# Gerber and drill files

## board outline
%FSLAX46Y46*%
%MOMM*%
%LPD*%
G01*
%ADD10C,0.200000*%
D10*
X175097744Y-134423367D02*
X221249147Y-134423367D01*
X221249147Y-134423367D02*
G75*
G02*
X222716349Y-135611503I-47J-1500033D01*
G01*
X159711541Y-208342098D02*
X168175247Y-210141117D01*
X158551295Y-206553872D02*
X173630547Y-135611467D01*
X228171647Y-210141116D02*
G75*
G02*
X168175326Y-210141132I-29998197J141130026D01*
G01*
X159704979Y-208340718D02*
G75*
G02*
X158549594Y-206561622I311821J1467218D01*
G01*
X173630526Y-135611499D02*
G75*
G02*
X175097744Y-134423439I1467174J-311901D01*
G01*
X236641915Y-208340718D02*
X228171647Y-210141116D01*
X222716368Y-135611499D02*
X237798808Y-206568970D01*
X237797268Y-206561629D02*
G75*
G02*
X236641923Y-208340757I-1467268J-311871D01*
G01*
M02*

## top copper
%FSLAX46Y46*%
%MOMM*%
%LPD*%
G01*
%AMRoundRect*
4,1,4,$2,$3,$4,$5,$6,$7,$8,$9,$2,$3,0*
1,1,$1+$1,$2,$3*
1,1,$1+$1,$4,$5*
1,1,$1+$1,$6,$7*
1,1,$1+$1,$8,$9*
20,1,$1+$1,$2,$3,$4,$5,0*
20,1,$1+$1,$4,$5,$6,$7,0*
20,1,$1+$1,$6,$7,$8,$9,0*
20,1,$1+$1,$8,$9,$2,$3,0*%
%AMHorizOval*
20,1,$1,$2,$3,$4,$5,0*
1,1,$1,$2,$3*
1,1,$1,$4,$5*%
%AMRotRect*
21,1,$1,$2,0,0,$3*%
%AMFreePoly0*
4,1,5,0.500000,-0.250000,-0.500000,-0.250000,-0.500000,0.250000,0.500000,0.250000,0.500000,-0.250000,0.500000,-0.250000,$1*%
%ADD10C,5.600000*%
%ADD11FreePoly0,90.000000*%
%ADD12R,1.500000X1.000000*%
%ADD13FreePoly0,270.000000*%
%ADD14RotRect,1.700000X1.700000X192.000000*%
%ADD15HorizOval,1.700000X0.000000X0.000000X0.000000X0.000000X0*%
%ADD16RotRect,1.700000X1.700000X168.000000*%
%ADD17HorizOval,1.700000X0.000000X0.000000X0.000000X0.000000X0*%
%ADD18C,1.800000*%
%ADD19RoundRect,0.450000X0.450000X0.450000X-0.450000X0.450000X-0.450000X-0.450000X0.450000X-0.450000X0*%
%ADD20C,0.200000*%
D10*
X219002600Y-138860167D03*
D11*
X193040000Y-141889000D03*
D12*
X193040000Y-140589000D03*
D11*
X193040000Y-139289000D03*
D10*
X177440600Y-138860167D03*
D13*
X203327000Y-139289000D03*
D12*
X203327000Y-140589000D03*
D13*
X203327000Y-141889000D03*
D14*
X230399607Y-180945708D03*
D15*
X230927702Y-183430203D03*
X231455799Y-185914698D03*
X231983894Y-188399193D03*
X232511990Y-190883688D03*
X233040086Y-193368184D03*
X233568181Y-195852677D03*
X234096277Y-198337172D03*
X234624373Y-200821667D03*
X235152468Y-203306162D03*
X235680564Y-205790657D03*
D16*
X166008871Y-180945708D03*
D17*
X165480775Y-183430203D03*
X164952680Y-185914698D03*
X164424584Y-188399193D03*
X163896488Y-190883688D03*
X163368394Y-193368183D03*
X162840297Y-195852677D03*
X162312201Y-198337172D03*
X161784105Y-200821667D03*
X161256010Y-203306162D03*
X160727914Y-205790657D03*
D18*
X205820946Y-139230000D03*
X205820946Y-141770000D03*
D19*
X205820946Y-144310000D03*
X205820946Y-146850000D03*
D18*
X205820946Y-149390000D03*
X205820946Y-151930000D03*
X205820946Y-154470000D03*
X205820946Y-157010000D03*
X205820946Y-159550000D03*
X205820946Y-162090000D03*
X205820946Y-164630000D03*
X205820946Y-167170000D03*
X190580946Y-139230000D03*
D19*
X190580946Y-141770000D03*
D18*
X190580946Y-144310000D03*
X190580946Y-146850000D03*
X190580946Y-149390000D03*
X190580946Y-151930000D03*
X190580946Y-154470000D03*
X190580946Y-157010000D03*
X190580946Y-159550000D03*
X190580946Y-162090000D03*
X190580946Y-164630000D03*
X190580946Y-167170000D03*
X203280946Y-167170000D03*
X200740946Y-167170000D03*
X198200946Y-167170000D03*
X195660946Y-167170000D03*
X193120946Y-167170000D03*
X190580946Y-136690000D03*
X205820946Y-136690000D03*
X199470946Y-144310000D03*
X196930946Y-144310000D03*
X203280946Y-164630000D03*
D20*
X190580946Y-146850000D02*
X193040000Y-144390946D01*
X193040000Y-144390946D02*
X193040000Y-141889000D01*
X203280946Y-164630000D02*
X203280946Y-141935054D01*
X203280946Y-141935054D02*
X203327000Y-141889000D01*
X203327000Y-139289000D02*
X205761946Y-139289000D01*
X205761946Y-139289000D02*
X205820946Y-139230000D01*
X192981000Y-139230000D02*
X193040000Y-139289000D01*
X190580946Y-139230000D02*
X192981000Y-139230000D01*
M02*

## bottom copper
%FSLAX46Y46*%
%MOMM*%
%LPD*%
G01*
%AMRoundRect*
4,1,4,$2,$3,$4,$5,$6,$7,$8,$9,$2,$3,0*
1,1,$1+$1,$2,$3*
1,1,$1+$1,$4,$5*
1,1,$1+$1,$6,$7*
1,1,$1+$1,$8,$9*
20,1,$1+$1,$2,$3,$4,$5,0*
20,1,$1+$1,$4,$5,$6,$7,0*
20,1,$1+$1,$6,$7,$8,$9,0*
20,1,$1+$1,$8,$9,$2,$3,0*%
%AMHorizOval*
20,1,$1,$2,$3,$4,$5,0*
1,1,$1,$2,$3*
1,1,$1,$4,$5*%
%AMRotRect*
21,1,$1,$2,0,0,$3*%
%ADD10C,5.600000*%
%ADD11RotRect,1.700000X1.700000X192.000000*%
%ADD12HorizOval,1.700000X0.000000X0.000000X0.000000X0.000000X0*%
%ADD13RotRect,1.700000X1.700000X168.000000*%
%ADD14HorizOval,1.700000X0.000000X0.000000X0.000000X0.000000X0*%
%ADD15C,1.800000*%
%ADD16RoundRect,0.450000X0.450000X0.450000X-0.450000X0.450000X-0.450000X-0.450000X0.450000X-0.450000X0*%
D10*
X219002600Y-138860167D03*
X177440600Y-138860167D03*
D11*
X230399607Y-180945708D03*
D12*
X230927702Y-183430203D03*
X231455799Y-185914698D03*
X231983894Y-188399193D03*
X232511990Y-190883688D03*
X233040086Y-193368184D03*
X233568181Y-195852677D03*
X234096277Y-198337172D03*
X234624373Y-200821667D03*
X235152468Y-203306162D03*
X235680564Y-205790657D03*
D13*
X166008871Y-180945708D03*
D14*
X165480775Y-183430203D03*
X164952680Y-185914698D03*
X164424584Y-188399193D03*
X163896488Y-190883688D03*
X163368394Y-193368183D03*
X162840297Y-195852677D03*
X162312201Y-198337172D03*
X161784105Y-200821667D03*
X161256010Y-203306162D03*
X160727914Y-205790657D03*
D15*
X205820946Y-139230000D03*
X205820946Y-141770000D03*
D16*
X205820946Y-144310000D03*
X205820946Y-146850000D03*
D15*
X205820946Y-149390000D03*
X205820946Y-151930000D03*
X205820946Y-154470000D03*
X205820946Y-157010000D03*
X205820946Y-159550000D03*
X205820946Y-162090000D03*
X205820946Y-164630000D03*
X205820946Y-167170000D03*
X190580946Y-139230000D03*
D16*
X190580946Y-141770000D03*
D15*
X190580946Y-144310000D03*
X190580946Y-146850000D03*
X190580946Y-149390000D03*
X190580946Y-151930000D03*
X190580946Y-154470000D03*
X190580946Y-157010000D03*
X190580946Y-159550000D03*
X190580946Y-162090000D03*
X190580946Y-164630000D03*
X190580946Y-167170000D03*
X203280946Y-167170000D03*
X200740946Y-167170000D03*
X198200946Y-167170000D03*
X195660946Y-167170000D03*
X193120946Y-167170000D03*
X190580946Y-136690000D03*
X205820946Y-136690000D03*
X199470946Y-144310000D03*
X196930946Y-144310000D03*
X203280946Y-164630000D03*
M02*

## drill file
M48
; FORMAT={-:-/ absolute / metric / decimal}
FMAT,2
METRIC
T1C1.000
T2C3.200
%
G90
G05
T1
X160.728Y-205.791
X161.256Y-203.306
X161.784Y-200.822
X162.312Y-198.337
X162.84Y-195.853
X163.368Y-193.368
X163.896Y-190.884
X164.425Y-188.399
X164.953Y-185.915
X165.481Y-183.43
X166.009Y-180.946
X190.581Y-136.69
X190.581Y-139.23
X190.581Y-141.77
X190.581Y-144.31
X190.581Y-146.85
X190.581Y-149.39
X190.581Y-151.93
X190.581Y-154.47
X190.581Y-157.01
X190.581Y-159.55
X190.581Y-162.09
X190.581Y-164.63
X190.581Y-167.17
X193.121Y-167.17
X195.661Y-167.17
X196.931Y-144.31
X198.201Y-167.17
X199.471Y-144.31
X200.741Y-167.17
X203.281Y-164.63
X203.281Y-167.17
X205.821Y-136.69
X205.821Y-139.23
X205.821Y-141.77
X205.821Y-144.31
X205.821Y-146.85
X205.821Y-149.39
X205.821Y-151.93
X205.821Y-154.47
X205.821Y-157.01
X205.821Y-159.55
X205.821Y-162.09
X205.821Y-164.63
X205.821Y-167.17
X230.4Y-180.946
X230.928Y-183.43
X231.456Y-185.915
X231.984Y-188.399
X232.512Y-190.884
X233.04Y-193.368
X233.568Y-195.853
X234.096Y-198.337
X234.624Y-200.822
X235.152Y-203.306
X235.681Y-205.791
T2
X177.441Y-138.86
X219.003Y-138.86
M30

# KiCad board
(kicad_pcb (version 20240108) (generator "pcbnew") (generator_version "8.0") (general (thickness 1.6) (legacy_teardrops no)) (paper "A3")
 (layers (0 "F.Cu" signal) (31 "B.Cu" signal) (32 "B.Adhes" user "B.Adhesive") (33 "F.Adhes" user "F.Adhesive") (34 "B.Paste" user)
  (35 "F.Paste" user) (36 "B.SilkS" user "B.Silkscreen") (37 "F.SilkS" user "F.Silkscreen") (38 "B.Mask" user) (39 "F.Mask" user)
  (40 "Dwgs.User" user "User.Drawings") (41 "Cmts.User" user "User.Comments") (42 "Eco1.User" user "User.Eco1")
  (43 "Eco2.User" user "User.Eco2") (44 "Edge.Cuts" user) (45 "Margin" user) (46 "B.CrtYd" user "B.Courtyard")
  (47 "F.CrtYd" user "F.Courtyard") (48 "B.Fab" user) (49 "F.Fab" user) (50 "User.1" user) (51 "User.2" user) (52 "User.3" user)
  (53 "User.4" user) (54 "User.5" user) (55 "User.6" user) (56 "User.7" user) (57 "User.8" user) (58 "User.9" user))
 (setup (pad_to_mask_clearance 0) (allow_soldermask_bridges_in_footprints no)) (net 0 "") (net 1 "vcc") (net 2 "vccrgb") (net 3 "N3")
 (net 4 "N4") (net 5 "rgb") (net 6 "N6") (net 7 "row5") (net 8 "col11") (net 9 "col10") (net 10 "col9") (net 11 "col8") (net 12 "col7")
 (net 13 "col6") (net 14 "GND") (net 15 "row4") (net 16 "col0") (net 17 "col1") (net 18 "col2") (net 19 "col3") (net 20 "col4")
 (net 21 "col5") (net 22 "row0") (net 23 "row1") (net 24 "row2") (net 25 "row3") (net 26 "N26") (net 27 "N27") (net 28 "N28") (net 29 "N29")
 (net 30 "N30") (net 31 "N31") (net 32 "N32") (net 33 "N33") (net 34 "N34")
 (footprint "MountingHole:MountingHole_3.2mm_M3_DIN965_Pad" (layer "F.Cu") (at 219.0026 138.860167)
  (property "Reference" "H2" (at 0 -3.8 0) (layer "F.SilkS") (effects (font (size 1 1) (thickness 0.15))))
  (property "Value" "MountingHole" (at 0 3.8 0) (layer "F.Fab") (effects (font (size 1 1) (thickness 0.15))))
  (pad "1" thru_hole circle (at 0 0) (size 5.6 5.6) (drill 3.2) (layers "*.Cu" "*.Mask") (remove_unused_layers no)))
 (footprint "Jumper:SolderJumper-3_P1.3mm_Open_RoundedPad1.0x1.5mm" (layer "F.Cu") (at 193.04 140.589 90)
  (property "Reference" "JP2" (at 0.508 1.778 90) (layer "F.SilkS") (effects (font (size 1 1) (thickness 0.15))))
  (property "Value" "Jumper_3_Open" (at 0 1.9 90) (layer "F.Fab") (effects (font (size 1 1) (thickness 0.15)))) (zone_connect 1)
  (pad "1" smd custom (at -1.3 0 90) (size 1 0.5) (layers "F.Cu" "F.Mask") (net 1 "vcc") (zone_connect 2) (thermal_bridge_angle 45)
   (options (clearance outline) (anchor rect)) (primitives))
  (pad "2" smd rect (at 0 0 90) (size 1 1.5) (layers "F.Cu" "F.Mask") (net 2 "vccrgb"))
  (pad "3" smd custom (at 1.3 0 90) (size 1 0.5) (layers "F.Cu" "F.Mask") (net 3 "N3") (zone_connect 2) (thermal_bridge_angle 45)
   (options (clearance outline) (anchor rect)) (primitives)))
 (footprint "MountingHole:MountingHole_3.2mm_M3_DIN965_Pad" (layer "F.Cu") (at 177.4406 138.860167)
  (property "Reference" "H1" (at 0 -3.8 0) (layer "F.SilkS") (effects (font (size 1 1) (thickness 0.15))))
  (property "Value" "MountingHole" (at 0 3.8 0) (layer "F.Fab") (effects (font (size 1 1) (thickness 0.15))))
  (pad "1" thru_hole circle (at 0 0) (size 5.6 5.6) (drill 3.2) (layers "*.Cu" "*.Mask") (remove_unused_layers no)))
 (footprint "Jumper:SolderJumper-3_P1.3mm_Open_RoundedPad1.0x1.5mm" (layer "F.Cu") (at 203.327 140.589 -90)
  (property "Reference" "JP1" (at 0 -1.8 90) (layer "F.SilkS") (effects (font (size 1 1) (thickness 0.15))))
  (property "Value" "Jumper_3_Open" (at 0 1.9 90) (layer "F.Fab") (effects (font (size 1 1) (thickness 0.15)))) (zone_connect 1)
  (pad "1" smd custom (at -1.3 0 270) (size 1 0.5) (layers "F.Cu" "F.Mask") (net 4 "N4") (zone_connect 2) (thermal_bridge_angle 45)
   (options (clearance outline) (anchor rect)) (primitives))
  (pad "2" smd rect (at 0 0 270) (size 1 1.5) (layers "F.Cu" "F.Mask") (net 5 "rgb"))
  (pad "3" smd custom (at 1.3 0 270) (size 1 0.5) (layers "F.Cu" "F.Mask") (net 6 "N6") (zone_connect 2) (thermal_bridge_angle 45)
   (options (clearance outline) (anchor rect)) (primitives)))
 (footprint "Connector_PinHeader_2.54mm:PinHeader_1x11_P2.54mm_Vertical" (layer "B.Cu") (at 230.399607 180.945708 -168)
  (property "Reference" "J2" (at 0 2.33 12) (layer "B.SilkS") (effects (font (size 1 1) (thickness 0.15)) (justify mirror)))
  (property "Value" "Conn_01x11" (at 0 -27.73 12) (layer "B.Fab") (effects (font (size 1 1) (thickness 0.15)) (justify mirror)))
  (pad "1" thru_hole rect (at 0 0 192) (size 1.7 1.7) (drill 1) (layers "*.Cu" "*.Mask") (remove_unused_layers no) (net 5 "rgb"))
  (pad "2" thru_hole oval (at 0.000001 -2.54 192) (size 1.7 1.7) (drill 1) (layers "*.Cu" "*.Mask") (remove_unused_layers no) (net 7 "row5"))
  (pad "3" thru_hole oval (at -0.000001 -5.08 192) (size 1.7 1.7) (drill 1) (layers "*.Cu" "*.Mask") (remove_unused_layers no)
   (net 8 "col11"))
  (pad "4" thru_hole oval (at 0 -7.62 192) (size 1.7 1.7) (drill 1) (layers "*.Cu" "*.Mask") (remove_unused_layers no) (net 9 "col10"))
  (pad "5" thru_hole oval (at 0 -10.16 192) (size 1.7 1.7) (drill 1) (layers "*.Cu" "*.Mask") (remove_unused_layers no) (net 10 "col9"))
  (pad "6" thru_hole oval (at 0 -12.700002 192) (size 1.7 1.7) (drill 1) (layers "*.Cu" "*.Mask") (remove_unused_layers no) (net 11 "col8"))
  (pad "7" thru_hole oval (at 0 -15.24 192) (size 1.7 1.7) (drill 1) (layers "*.Cu" "*.Mask") (remove_unused_layers no) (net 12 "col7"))
  (pad "8" thru_hole oval (at 0 -17.78 192) (size 1.7 1.7) (drill 1) (layers "*.Cu" "*.Mask") (remove_unused_layers no) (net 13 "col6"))
  (pad "9" thru_hole oval (at 0 -20.32 192) (size 1.7 1.7) (drill 1) (layers "*.Cu" "*.Mask") (remove_unused_layers no) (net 2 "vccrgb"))
  (pad "10" thru_hole oval (at 0 -22.86 192) (size 1.7 1.7) (drill 1) (layers "*.Cu" "*.Mask") (remove_unused_layers no) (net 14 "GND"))
  (pad "11" thru_hole oval (at 0 -25.4 192) (size 1.7 1.7) (drill 1) (layers "*.Cu" "*.Mask") (remove_unused_layers no) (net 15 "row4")))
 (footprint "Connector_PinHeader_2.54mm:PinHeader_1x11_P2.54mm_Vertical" (layer "B.Cu") (at 166.008871 180.945708 168)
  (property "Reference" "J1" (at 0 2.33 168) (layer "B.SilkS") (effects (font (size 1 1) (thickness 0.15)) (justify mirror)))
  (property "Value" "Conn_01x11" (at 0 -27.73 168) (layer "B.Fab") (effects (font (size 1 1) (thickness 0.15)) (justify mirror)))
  (pad "1" thru_hole rect (at 0 0 168) (size 1.7 1.7) (drill 1) (layers "*.Cu" "*.Mask") (remove_unused_layers no) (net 14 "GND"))
  (pad "2" thru_hole oval (at 0 -2.54 168) (size 1.7 1.7) (drill 1) (layers "*.Cu" "*.Mask") (remove_unused_layers no) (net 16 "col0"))
  (pad "3" thru_hole oval (at 0 -5.08 168) (size 1.7 1.7) (drill 1) (layers "*.Cu" "*.Mask") (remove_unused_layers no) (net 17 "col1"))
  (pad "4" thru_hole oval (at 0 -7.62 168) (size 1.7 1.7) (drill 1) (layers "*.Cu" "*.Mask") (remove_unused_layers no) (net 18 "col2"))
  (pad "5" thru_hole oval (at 0 -10.16 168) (size 1.7 1.7) (drill 1) (layers "*.Cu" "*.Mask") (remove_unused_layers no) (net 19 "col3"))
  (pad "6" thru_hole oval (at -0.000002 -12.7 168) (size 1.7 1.7) (drill 1) (layers "*.Cu" "*.Mask") (remove_unused_layers no)
   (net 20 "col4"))
  (pad "7" thru_hole oval (at 0 -15.24 168) (size 1.7 1.7) (drill 1) (layers "*.Cu" "*.Mask") (remove_unused_layers no) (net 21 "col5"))
  (pad "8" thru_hole oval (at 0 -17.78 168) (size 1.7 1.7) (drill 1) (layers "*.Cu" "*.Mask") (remove_unused_layers no) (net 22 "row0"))
  (pad "9" thru_hole oval (at 0 -20.32 168) (size 1.7 1.7) (drill 1) (layers "*.Cu" "*.Mask") (remove_unused_layers no) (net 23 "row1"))
  (pad "10" thru_hole oval (at 0 -22.86 168) (size 1.7 1.7) (drill 1) (layers "*.Cu" "*.Mask") (remove_unused_layers no) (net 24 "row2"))
  (pad "11" thru_hole oval (at 0 -25.4 168) (size 1.7 1.7) (drill 1) (layers "*.Cu" "*.Mask") (remove_unused_layers no) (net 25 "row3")))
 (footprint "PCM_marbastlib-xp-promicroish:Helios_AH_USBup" (layer "B.Cu") (at 198.200946 153.2 180)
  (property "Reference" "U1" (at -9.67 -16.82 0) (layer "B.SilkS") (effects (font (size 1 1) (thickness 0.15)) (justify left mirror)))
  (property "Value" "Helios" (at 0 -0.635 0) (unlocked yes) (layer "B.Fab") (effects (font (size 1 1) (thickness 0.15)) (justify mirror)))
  (pad "1" thru_hole circle (at -7.62 13.97 180) (size 1.8 1.8) (drill 1) (layers "*.Cu" "F.Mask") (remove_unused_layers no) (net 4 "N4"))
  (pad "2" thru_hole circle (at -7.62 11.43 180) (size 1.8 1.8) (drill 1) (layers "*.Cu" "F.Mask") (remove_unused_layers no) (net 8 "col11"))
  (pad "3" thru_hole roundrect (at -7.62 8.89 180) (size 1.8 1.8) (drill 1) (layers "*.Cu" "F.Mask") (remove_unused_layers no)
   (roundrect_rratio 0.25) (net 14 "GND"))
  (pad "4" thru_hole roundrect (at -7.62 6.35 180) (size 1.8 1.8) (drill 1) (layers "*.Cu" "F.Mask") (remove_unused_layers no)
   (roundrect_rratio 0.25) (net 14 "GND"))
  (pad "5" thru_hole circle (at -7.62 3.81 180) (size 1.8 1.8) (drill 1) (layers "*.Cu" "F.Mask") (remove_unused_layers no) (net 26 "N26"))
  (pad "6" thru_hole circle (at -7.62 1.27 180) (size 1.8 1.8) (drill 1) (layers "*.Cu" "F.Mask") (remove_unused_layers no) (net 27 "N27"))
  (pad "7" thru_hole circle (at -7.62 -1.27 180) (size 1.8 1.8) (drill 1) (layers "*.Cu" "F.Mask") (remove_unused_layers no) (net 9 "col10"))
  (pad "8" thru_hole circle (at -7.62 -3.81 180) (size 1.8 1.8) (drill 1) (layers "*.Cu" "F.Mask") (remove_unused_layers no) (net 10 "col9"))
  (pad "9" thru_hole circle (at -7.62 -6.35 180) (size 1.8 1.8) (drill 1) (layers "*.Cu" "F.Mask") (remove_unused_layers no) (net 11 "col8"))
  (pad "10" thru_hole circle (at -7.62 -8.89 180) (size 1.8 1.8) (drill 1) (layers "*.Cu" "F.Mask") (remove_unused_layers no)
   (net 12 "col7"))
  (pad "11" thru_hole circle (at -7.62 -11.43 180) (size 1.8 1.8) (drill 1) (layers "*.Cu" "F.Mask") (remove_unused_layers no)
   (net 13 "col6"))
  (pad "12" thru_hole circle (at -7.62 -13.97 180) (size 1.8 1.8) (drill 1) (layers "*.Cu" "F.Mask") (remove_unused_layers no)
   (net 15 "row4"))
  (pad "13" thru_hole circle (at 7.62 13.97 180) (size 1.8 1.8) (drill 1) (layers "*.Cu" "F.Mask") (remove_unused_layers no) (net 3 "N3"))
  (pad "14" thru_hole roundrect (at 7.62 11.43 180) (size 1.8 1.8) (drill 1) (layers "*.Cu" "F.Mask") (remove_unused_layers no)
   (roundrect_rratio 0.25) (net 14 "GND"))
  (pad "15" thru_hole circle (at 7.62 8.89 180) (size 1.8 1.8) (drill 1) (layers "*.Cu" "F.Mask") (remove_unused_layers no) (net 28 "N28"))
  (pad "16" thru_hole circle (at 7.62 6.35 180) (size 1.8 1.8) (drill 1) (layers "*.Cu" "F.Mask") (remove_unused_layers no) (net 1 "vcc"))
  (pad "17" thru_hole circle (at 7.62 3.81 180) (size 1.8 1.8) (drill 1) (layers "*.Cu" "F.Mask") (remove_unused_layers no) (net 17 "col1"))
  (pad "18" thru_hole circle (at 7.62 1.27 180) (size 1.8 1.8) (drill 1) (layers "*.Cu" "F.Mask") (remove_unused_layers no) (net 18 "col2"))
  (pad "19" thru_hole circle (at 7.62 -1.27 180) (size 1.8 1.8) (drill 1) (layers "*.Cu" "F.Mask") (remove_unused_layers no) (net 19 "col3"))
  (pad "20" thru_hole circle (at 7.62 -3.81 180) (size 1.8 1.8) (drill 1) (layers "*.Cu" "F.Mask") (remove_unused_layers no) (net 20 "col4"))
  (pad "21" thru_hole circle (at 7.62 -6.35 180) (size 1.8 1.8) (drill 1) (layers "*.Cu" "F.Mask") (remove_unused_layers no) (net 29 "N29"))
  (pad "22" thru_hole circle (at 7.62 -8.89 180) (size 1.8 1.8) (drill 1) (layers "*.Cu" "F.Mask") (remove_unused_layers no) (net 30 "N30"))
  (pad "23" thru_hole circle (at 7.62 -11.43 180) (size 1.8 1.8) (drill 1) (layers "*.Cu" "F.Mask") (remove_unused_layers no) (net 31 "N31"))
  (pad "24" thru_hole circle (at 7.62 -13.97 180) (size 1.8 1.8) (drill 1) (layers "*.Cu" "F.Mask") (remove_unused_layers no) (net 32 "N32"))
  (pad "25" thru_hole circle (at -5.08 -13.97 180) (size 1.8 1.8) (drill 1) (layers "*.Cu" "F.Mask") (remove_unused_layers no)
   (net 25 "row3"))
  (pad "26" thru_hole circle (at -2.54 -13.97 180) (size 1.8 1.8) (drill 1) (layers "*.Cu" "F.Mask") (remove_unused_layers no)
   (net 24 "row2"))
  (pad "27" thru_hole circle (at 0 -13.97 180) (size 1.8 1.8) (drill 1) (layers "*.Cu" "F.Mask") (remove_unused_layers no) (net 23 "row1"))
  (pad "28" thru_hole circle (at 2.54 -13.97 180) (size 1.8 1.8) (drill 1) (layers "*.Cu" "F.Mask") (remove_unused_layers no)
   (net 22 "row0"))
  (pad "29" thru_hole circle (at 5.08 -13.97 180) (size 1.8 1.8) (drill 1) (layers "*.Cu" "F.Mask") (remove_unused_layers no)
   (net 21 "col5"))
  (pad "30" thru_hole circle (at 7.62 16.51 180) (size 1.8 1.8) (drill 1) (layers "*.Cu" "F.Mask") (remove_unused_layers no) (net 16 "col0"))
  (pad "31" thru_hole circle (at -7.62 16.51 180) (size 1.8 1.8) (drill 1) (layers "*.Cu" "F.Mask") (remove_unused_layers no) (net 7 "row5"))
  (pad "32" thru_hole circle (at -1.27 8.89 180) (size 1.8 1.8) (drill 1) (layers "*.Cu" "F.Mask") (remove_unused_layers no) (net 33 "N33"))
  (pad "33" thru_hole circle (at 1.27 8.89 180) (size 1.8 1.8) (drill 1) (layers "*.Cu" "F.Mask") (remove_unused_layers no) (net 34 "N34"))
  (pad "34" thru_hole circle (at -5.08 -11.43 180) (size 1.8 1.8) (drill 1) (layers "*.Cu" "F.Mask") (remove_unused_layers no) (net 6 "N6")))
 (gr_line (start 175.097744 134.423367) (end 221.249147 134.423367) (stroke (width 0.2) (type default)) (layer "Edge.Cuts"))
 (gr_arc (start 221.249147 134.423367) (mid 222.193127 134.757648) (end 222.716368 135.611499) (stroke (width 0.2) (type default))
  (layer "Edge.Cuts"))
 (gr_line (start 159.711541 208.342098) (end 168.175247 210.141117) (stroke (width 0.2) (type default)) (layer "Edge.Cuts"))
 (gr_line (start 158.551295 206.553872) (end 173.630547 135.611467) (stroke (width 0.2) (type default)) (layer "Edge.Cuts"))
 (gr_arc (start 228.171647 210.141116) (mid 198.173487 213.294063) (end 168.175326 210.141133) (stroke (width 0.2) (type default))
  (layer "Edge.Cuts"))
 (gr_arc (start 159.704979 208.340718) (mid 158.75884 207.690455) (end 158.549626 206.561629) (stroke (width 0.2) (type default))
  (layer "Edge.Cuts"))
 (gr_arc (start 173.630526 135.611499) (mid 174.153765 134.757648) (end 175.097744 134.423367) (stroke (width 0.2) (type default))
  (layer "Edge.Cuts"))
 (gr_line (start 236.641915 208.340718) (end 228.171647 210.141116) (stroke (width 0.2) (type default)) (layer "Edge.Cuts"))
 (gr_line (start 222.716368 135.611499) (end 237.798808 206.56897) (stroke (width 0.2) (type default)) (layer "Edge.Cuts"))
 (gr_arc (start 237.797268 206.561629) (mid 237.588038 207.690436) (end 236.641915 208.340718) (stroke (width 0.2) (type default))
  (layer "Edge.Cuts"))
 (segment (start 190.580946 146.85) (end 193.04 144.390946) (width 0.2) (layer "F.Cu") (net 1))
 (segment (start 193.04 144.390946) (end 193.04 141.889) (width 0.2) (layer "F.Cu") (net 1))
 (segment (start 203.280946 164.63) (end 203.280946 141.935054) (width 0.2) (layer "F.Cu") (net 6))
 (segment (start 203.280946 141.935054) (end 203.327 141.889) (width 0.2) (layer "F.Cu") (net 6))
 (segment (start 203.327 139.289) (end 205.761946 139.289) (width 0.2) (layer "F.Cu") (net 4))
 (segment (start 205.761946 139.289) (end 205.820946 139.23) (width 0.2) (layer "F.Cu") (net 4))
 (segment (start 192.981 139.23) (end 193.04 139.289) (width 0.2) (layer "F.Cu") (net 3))
 (segment (start 190.580946 139.23) (end 192.981 139.23) (width 0.2) (layer "F.Cu") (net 3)))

